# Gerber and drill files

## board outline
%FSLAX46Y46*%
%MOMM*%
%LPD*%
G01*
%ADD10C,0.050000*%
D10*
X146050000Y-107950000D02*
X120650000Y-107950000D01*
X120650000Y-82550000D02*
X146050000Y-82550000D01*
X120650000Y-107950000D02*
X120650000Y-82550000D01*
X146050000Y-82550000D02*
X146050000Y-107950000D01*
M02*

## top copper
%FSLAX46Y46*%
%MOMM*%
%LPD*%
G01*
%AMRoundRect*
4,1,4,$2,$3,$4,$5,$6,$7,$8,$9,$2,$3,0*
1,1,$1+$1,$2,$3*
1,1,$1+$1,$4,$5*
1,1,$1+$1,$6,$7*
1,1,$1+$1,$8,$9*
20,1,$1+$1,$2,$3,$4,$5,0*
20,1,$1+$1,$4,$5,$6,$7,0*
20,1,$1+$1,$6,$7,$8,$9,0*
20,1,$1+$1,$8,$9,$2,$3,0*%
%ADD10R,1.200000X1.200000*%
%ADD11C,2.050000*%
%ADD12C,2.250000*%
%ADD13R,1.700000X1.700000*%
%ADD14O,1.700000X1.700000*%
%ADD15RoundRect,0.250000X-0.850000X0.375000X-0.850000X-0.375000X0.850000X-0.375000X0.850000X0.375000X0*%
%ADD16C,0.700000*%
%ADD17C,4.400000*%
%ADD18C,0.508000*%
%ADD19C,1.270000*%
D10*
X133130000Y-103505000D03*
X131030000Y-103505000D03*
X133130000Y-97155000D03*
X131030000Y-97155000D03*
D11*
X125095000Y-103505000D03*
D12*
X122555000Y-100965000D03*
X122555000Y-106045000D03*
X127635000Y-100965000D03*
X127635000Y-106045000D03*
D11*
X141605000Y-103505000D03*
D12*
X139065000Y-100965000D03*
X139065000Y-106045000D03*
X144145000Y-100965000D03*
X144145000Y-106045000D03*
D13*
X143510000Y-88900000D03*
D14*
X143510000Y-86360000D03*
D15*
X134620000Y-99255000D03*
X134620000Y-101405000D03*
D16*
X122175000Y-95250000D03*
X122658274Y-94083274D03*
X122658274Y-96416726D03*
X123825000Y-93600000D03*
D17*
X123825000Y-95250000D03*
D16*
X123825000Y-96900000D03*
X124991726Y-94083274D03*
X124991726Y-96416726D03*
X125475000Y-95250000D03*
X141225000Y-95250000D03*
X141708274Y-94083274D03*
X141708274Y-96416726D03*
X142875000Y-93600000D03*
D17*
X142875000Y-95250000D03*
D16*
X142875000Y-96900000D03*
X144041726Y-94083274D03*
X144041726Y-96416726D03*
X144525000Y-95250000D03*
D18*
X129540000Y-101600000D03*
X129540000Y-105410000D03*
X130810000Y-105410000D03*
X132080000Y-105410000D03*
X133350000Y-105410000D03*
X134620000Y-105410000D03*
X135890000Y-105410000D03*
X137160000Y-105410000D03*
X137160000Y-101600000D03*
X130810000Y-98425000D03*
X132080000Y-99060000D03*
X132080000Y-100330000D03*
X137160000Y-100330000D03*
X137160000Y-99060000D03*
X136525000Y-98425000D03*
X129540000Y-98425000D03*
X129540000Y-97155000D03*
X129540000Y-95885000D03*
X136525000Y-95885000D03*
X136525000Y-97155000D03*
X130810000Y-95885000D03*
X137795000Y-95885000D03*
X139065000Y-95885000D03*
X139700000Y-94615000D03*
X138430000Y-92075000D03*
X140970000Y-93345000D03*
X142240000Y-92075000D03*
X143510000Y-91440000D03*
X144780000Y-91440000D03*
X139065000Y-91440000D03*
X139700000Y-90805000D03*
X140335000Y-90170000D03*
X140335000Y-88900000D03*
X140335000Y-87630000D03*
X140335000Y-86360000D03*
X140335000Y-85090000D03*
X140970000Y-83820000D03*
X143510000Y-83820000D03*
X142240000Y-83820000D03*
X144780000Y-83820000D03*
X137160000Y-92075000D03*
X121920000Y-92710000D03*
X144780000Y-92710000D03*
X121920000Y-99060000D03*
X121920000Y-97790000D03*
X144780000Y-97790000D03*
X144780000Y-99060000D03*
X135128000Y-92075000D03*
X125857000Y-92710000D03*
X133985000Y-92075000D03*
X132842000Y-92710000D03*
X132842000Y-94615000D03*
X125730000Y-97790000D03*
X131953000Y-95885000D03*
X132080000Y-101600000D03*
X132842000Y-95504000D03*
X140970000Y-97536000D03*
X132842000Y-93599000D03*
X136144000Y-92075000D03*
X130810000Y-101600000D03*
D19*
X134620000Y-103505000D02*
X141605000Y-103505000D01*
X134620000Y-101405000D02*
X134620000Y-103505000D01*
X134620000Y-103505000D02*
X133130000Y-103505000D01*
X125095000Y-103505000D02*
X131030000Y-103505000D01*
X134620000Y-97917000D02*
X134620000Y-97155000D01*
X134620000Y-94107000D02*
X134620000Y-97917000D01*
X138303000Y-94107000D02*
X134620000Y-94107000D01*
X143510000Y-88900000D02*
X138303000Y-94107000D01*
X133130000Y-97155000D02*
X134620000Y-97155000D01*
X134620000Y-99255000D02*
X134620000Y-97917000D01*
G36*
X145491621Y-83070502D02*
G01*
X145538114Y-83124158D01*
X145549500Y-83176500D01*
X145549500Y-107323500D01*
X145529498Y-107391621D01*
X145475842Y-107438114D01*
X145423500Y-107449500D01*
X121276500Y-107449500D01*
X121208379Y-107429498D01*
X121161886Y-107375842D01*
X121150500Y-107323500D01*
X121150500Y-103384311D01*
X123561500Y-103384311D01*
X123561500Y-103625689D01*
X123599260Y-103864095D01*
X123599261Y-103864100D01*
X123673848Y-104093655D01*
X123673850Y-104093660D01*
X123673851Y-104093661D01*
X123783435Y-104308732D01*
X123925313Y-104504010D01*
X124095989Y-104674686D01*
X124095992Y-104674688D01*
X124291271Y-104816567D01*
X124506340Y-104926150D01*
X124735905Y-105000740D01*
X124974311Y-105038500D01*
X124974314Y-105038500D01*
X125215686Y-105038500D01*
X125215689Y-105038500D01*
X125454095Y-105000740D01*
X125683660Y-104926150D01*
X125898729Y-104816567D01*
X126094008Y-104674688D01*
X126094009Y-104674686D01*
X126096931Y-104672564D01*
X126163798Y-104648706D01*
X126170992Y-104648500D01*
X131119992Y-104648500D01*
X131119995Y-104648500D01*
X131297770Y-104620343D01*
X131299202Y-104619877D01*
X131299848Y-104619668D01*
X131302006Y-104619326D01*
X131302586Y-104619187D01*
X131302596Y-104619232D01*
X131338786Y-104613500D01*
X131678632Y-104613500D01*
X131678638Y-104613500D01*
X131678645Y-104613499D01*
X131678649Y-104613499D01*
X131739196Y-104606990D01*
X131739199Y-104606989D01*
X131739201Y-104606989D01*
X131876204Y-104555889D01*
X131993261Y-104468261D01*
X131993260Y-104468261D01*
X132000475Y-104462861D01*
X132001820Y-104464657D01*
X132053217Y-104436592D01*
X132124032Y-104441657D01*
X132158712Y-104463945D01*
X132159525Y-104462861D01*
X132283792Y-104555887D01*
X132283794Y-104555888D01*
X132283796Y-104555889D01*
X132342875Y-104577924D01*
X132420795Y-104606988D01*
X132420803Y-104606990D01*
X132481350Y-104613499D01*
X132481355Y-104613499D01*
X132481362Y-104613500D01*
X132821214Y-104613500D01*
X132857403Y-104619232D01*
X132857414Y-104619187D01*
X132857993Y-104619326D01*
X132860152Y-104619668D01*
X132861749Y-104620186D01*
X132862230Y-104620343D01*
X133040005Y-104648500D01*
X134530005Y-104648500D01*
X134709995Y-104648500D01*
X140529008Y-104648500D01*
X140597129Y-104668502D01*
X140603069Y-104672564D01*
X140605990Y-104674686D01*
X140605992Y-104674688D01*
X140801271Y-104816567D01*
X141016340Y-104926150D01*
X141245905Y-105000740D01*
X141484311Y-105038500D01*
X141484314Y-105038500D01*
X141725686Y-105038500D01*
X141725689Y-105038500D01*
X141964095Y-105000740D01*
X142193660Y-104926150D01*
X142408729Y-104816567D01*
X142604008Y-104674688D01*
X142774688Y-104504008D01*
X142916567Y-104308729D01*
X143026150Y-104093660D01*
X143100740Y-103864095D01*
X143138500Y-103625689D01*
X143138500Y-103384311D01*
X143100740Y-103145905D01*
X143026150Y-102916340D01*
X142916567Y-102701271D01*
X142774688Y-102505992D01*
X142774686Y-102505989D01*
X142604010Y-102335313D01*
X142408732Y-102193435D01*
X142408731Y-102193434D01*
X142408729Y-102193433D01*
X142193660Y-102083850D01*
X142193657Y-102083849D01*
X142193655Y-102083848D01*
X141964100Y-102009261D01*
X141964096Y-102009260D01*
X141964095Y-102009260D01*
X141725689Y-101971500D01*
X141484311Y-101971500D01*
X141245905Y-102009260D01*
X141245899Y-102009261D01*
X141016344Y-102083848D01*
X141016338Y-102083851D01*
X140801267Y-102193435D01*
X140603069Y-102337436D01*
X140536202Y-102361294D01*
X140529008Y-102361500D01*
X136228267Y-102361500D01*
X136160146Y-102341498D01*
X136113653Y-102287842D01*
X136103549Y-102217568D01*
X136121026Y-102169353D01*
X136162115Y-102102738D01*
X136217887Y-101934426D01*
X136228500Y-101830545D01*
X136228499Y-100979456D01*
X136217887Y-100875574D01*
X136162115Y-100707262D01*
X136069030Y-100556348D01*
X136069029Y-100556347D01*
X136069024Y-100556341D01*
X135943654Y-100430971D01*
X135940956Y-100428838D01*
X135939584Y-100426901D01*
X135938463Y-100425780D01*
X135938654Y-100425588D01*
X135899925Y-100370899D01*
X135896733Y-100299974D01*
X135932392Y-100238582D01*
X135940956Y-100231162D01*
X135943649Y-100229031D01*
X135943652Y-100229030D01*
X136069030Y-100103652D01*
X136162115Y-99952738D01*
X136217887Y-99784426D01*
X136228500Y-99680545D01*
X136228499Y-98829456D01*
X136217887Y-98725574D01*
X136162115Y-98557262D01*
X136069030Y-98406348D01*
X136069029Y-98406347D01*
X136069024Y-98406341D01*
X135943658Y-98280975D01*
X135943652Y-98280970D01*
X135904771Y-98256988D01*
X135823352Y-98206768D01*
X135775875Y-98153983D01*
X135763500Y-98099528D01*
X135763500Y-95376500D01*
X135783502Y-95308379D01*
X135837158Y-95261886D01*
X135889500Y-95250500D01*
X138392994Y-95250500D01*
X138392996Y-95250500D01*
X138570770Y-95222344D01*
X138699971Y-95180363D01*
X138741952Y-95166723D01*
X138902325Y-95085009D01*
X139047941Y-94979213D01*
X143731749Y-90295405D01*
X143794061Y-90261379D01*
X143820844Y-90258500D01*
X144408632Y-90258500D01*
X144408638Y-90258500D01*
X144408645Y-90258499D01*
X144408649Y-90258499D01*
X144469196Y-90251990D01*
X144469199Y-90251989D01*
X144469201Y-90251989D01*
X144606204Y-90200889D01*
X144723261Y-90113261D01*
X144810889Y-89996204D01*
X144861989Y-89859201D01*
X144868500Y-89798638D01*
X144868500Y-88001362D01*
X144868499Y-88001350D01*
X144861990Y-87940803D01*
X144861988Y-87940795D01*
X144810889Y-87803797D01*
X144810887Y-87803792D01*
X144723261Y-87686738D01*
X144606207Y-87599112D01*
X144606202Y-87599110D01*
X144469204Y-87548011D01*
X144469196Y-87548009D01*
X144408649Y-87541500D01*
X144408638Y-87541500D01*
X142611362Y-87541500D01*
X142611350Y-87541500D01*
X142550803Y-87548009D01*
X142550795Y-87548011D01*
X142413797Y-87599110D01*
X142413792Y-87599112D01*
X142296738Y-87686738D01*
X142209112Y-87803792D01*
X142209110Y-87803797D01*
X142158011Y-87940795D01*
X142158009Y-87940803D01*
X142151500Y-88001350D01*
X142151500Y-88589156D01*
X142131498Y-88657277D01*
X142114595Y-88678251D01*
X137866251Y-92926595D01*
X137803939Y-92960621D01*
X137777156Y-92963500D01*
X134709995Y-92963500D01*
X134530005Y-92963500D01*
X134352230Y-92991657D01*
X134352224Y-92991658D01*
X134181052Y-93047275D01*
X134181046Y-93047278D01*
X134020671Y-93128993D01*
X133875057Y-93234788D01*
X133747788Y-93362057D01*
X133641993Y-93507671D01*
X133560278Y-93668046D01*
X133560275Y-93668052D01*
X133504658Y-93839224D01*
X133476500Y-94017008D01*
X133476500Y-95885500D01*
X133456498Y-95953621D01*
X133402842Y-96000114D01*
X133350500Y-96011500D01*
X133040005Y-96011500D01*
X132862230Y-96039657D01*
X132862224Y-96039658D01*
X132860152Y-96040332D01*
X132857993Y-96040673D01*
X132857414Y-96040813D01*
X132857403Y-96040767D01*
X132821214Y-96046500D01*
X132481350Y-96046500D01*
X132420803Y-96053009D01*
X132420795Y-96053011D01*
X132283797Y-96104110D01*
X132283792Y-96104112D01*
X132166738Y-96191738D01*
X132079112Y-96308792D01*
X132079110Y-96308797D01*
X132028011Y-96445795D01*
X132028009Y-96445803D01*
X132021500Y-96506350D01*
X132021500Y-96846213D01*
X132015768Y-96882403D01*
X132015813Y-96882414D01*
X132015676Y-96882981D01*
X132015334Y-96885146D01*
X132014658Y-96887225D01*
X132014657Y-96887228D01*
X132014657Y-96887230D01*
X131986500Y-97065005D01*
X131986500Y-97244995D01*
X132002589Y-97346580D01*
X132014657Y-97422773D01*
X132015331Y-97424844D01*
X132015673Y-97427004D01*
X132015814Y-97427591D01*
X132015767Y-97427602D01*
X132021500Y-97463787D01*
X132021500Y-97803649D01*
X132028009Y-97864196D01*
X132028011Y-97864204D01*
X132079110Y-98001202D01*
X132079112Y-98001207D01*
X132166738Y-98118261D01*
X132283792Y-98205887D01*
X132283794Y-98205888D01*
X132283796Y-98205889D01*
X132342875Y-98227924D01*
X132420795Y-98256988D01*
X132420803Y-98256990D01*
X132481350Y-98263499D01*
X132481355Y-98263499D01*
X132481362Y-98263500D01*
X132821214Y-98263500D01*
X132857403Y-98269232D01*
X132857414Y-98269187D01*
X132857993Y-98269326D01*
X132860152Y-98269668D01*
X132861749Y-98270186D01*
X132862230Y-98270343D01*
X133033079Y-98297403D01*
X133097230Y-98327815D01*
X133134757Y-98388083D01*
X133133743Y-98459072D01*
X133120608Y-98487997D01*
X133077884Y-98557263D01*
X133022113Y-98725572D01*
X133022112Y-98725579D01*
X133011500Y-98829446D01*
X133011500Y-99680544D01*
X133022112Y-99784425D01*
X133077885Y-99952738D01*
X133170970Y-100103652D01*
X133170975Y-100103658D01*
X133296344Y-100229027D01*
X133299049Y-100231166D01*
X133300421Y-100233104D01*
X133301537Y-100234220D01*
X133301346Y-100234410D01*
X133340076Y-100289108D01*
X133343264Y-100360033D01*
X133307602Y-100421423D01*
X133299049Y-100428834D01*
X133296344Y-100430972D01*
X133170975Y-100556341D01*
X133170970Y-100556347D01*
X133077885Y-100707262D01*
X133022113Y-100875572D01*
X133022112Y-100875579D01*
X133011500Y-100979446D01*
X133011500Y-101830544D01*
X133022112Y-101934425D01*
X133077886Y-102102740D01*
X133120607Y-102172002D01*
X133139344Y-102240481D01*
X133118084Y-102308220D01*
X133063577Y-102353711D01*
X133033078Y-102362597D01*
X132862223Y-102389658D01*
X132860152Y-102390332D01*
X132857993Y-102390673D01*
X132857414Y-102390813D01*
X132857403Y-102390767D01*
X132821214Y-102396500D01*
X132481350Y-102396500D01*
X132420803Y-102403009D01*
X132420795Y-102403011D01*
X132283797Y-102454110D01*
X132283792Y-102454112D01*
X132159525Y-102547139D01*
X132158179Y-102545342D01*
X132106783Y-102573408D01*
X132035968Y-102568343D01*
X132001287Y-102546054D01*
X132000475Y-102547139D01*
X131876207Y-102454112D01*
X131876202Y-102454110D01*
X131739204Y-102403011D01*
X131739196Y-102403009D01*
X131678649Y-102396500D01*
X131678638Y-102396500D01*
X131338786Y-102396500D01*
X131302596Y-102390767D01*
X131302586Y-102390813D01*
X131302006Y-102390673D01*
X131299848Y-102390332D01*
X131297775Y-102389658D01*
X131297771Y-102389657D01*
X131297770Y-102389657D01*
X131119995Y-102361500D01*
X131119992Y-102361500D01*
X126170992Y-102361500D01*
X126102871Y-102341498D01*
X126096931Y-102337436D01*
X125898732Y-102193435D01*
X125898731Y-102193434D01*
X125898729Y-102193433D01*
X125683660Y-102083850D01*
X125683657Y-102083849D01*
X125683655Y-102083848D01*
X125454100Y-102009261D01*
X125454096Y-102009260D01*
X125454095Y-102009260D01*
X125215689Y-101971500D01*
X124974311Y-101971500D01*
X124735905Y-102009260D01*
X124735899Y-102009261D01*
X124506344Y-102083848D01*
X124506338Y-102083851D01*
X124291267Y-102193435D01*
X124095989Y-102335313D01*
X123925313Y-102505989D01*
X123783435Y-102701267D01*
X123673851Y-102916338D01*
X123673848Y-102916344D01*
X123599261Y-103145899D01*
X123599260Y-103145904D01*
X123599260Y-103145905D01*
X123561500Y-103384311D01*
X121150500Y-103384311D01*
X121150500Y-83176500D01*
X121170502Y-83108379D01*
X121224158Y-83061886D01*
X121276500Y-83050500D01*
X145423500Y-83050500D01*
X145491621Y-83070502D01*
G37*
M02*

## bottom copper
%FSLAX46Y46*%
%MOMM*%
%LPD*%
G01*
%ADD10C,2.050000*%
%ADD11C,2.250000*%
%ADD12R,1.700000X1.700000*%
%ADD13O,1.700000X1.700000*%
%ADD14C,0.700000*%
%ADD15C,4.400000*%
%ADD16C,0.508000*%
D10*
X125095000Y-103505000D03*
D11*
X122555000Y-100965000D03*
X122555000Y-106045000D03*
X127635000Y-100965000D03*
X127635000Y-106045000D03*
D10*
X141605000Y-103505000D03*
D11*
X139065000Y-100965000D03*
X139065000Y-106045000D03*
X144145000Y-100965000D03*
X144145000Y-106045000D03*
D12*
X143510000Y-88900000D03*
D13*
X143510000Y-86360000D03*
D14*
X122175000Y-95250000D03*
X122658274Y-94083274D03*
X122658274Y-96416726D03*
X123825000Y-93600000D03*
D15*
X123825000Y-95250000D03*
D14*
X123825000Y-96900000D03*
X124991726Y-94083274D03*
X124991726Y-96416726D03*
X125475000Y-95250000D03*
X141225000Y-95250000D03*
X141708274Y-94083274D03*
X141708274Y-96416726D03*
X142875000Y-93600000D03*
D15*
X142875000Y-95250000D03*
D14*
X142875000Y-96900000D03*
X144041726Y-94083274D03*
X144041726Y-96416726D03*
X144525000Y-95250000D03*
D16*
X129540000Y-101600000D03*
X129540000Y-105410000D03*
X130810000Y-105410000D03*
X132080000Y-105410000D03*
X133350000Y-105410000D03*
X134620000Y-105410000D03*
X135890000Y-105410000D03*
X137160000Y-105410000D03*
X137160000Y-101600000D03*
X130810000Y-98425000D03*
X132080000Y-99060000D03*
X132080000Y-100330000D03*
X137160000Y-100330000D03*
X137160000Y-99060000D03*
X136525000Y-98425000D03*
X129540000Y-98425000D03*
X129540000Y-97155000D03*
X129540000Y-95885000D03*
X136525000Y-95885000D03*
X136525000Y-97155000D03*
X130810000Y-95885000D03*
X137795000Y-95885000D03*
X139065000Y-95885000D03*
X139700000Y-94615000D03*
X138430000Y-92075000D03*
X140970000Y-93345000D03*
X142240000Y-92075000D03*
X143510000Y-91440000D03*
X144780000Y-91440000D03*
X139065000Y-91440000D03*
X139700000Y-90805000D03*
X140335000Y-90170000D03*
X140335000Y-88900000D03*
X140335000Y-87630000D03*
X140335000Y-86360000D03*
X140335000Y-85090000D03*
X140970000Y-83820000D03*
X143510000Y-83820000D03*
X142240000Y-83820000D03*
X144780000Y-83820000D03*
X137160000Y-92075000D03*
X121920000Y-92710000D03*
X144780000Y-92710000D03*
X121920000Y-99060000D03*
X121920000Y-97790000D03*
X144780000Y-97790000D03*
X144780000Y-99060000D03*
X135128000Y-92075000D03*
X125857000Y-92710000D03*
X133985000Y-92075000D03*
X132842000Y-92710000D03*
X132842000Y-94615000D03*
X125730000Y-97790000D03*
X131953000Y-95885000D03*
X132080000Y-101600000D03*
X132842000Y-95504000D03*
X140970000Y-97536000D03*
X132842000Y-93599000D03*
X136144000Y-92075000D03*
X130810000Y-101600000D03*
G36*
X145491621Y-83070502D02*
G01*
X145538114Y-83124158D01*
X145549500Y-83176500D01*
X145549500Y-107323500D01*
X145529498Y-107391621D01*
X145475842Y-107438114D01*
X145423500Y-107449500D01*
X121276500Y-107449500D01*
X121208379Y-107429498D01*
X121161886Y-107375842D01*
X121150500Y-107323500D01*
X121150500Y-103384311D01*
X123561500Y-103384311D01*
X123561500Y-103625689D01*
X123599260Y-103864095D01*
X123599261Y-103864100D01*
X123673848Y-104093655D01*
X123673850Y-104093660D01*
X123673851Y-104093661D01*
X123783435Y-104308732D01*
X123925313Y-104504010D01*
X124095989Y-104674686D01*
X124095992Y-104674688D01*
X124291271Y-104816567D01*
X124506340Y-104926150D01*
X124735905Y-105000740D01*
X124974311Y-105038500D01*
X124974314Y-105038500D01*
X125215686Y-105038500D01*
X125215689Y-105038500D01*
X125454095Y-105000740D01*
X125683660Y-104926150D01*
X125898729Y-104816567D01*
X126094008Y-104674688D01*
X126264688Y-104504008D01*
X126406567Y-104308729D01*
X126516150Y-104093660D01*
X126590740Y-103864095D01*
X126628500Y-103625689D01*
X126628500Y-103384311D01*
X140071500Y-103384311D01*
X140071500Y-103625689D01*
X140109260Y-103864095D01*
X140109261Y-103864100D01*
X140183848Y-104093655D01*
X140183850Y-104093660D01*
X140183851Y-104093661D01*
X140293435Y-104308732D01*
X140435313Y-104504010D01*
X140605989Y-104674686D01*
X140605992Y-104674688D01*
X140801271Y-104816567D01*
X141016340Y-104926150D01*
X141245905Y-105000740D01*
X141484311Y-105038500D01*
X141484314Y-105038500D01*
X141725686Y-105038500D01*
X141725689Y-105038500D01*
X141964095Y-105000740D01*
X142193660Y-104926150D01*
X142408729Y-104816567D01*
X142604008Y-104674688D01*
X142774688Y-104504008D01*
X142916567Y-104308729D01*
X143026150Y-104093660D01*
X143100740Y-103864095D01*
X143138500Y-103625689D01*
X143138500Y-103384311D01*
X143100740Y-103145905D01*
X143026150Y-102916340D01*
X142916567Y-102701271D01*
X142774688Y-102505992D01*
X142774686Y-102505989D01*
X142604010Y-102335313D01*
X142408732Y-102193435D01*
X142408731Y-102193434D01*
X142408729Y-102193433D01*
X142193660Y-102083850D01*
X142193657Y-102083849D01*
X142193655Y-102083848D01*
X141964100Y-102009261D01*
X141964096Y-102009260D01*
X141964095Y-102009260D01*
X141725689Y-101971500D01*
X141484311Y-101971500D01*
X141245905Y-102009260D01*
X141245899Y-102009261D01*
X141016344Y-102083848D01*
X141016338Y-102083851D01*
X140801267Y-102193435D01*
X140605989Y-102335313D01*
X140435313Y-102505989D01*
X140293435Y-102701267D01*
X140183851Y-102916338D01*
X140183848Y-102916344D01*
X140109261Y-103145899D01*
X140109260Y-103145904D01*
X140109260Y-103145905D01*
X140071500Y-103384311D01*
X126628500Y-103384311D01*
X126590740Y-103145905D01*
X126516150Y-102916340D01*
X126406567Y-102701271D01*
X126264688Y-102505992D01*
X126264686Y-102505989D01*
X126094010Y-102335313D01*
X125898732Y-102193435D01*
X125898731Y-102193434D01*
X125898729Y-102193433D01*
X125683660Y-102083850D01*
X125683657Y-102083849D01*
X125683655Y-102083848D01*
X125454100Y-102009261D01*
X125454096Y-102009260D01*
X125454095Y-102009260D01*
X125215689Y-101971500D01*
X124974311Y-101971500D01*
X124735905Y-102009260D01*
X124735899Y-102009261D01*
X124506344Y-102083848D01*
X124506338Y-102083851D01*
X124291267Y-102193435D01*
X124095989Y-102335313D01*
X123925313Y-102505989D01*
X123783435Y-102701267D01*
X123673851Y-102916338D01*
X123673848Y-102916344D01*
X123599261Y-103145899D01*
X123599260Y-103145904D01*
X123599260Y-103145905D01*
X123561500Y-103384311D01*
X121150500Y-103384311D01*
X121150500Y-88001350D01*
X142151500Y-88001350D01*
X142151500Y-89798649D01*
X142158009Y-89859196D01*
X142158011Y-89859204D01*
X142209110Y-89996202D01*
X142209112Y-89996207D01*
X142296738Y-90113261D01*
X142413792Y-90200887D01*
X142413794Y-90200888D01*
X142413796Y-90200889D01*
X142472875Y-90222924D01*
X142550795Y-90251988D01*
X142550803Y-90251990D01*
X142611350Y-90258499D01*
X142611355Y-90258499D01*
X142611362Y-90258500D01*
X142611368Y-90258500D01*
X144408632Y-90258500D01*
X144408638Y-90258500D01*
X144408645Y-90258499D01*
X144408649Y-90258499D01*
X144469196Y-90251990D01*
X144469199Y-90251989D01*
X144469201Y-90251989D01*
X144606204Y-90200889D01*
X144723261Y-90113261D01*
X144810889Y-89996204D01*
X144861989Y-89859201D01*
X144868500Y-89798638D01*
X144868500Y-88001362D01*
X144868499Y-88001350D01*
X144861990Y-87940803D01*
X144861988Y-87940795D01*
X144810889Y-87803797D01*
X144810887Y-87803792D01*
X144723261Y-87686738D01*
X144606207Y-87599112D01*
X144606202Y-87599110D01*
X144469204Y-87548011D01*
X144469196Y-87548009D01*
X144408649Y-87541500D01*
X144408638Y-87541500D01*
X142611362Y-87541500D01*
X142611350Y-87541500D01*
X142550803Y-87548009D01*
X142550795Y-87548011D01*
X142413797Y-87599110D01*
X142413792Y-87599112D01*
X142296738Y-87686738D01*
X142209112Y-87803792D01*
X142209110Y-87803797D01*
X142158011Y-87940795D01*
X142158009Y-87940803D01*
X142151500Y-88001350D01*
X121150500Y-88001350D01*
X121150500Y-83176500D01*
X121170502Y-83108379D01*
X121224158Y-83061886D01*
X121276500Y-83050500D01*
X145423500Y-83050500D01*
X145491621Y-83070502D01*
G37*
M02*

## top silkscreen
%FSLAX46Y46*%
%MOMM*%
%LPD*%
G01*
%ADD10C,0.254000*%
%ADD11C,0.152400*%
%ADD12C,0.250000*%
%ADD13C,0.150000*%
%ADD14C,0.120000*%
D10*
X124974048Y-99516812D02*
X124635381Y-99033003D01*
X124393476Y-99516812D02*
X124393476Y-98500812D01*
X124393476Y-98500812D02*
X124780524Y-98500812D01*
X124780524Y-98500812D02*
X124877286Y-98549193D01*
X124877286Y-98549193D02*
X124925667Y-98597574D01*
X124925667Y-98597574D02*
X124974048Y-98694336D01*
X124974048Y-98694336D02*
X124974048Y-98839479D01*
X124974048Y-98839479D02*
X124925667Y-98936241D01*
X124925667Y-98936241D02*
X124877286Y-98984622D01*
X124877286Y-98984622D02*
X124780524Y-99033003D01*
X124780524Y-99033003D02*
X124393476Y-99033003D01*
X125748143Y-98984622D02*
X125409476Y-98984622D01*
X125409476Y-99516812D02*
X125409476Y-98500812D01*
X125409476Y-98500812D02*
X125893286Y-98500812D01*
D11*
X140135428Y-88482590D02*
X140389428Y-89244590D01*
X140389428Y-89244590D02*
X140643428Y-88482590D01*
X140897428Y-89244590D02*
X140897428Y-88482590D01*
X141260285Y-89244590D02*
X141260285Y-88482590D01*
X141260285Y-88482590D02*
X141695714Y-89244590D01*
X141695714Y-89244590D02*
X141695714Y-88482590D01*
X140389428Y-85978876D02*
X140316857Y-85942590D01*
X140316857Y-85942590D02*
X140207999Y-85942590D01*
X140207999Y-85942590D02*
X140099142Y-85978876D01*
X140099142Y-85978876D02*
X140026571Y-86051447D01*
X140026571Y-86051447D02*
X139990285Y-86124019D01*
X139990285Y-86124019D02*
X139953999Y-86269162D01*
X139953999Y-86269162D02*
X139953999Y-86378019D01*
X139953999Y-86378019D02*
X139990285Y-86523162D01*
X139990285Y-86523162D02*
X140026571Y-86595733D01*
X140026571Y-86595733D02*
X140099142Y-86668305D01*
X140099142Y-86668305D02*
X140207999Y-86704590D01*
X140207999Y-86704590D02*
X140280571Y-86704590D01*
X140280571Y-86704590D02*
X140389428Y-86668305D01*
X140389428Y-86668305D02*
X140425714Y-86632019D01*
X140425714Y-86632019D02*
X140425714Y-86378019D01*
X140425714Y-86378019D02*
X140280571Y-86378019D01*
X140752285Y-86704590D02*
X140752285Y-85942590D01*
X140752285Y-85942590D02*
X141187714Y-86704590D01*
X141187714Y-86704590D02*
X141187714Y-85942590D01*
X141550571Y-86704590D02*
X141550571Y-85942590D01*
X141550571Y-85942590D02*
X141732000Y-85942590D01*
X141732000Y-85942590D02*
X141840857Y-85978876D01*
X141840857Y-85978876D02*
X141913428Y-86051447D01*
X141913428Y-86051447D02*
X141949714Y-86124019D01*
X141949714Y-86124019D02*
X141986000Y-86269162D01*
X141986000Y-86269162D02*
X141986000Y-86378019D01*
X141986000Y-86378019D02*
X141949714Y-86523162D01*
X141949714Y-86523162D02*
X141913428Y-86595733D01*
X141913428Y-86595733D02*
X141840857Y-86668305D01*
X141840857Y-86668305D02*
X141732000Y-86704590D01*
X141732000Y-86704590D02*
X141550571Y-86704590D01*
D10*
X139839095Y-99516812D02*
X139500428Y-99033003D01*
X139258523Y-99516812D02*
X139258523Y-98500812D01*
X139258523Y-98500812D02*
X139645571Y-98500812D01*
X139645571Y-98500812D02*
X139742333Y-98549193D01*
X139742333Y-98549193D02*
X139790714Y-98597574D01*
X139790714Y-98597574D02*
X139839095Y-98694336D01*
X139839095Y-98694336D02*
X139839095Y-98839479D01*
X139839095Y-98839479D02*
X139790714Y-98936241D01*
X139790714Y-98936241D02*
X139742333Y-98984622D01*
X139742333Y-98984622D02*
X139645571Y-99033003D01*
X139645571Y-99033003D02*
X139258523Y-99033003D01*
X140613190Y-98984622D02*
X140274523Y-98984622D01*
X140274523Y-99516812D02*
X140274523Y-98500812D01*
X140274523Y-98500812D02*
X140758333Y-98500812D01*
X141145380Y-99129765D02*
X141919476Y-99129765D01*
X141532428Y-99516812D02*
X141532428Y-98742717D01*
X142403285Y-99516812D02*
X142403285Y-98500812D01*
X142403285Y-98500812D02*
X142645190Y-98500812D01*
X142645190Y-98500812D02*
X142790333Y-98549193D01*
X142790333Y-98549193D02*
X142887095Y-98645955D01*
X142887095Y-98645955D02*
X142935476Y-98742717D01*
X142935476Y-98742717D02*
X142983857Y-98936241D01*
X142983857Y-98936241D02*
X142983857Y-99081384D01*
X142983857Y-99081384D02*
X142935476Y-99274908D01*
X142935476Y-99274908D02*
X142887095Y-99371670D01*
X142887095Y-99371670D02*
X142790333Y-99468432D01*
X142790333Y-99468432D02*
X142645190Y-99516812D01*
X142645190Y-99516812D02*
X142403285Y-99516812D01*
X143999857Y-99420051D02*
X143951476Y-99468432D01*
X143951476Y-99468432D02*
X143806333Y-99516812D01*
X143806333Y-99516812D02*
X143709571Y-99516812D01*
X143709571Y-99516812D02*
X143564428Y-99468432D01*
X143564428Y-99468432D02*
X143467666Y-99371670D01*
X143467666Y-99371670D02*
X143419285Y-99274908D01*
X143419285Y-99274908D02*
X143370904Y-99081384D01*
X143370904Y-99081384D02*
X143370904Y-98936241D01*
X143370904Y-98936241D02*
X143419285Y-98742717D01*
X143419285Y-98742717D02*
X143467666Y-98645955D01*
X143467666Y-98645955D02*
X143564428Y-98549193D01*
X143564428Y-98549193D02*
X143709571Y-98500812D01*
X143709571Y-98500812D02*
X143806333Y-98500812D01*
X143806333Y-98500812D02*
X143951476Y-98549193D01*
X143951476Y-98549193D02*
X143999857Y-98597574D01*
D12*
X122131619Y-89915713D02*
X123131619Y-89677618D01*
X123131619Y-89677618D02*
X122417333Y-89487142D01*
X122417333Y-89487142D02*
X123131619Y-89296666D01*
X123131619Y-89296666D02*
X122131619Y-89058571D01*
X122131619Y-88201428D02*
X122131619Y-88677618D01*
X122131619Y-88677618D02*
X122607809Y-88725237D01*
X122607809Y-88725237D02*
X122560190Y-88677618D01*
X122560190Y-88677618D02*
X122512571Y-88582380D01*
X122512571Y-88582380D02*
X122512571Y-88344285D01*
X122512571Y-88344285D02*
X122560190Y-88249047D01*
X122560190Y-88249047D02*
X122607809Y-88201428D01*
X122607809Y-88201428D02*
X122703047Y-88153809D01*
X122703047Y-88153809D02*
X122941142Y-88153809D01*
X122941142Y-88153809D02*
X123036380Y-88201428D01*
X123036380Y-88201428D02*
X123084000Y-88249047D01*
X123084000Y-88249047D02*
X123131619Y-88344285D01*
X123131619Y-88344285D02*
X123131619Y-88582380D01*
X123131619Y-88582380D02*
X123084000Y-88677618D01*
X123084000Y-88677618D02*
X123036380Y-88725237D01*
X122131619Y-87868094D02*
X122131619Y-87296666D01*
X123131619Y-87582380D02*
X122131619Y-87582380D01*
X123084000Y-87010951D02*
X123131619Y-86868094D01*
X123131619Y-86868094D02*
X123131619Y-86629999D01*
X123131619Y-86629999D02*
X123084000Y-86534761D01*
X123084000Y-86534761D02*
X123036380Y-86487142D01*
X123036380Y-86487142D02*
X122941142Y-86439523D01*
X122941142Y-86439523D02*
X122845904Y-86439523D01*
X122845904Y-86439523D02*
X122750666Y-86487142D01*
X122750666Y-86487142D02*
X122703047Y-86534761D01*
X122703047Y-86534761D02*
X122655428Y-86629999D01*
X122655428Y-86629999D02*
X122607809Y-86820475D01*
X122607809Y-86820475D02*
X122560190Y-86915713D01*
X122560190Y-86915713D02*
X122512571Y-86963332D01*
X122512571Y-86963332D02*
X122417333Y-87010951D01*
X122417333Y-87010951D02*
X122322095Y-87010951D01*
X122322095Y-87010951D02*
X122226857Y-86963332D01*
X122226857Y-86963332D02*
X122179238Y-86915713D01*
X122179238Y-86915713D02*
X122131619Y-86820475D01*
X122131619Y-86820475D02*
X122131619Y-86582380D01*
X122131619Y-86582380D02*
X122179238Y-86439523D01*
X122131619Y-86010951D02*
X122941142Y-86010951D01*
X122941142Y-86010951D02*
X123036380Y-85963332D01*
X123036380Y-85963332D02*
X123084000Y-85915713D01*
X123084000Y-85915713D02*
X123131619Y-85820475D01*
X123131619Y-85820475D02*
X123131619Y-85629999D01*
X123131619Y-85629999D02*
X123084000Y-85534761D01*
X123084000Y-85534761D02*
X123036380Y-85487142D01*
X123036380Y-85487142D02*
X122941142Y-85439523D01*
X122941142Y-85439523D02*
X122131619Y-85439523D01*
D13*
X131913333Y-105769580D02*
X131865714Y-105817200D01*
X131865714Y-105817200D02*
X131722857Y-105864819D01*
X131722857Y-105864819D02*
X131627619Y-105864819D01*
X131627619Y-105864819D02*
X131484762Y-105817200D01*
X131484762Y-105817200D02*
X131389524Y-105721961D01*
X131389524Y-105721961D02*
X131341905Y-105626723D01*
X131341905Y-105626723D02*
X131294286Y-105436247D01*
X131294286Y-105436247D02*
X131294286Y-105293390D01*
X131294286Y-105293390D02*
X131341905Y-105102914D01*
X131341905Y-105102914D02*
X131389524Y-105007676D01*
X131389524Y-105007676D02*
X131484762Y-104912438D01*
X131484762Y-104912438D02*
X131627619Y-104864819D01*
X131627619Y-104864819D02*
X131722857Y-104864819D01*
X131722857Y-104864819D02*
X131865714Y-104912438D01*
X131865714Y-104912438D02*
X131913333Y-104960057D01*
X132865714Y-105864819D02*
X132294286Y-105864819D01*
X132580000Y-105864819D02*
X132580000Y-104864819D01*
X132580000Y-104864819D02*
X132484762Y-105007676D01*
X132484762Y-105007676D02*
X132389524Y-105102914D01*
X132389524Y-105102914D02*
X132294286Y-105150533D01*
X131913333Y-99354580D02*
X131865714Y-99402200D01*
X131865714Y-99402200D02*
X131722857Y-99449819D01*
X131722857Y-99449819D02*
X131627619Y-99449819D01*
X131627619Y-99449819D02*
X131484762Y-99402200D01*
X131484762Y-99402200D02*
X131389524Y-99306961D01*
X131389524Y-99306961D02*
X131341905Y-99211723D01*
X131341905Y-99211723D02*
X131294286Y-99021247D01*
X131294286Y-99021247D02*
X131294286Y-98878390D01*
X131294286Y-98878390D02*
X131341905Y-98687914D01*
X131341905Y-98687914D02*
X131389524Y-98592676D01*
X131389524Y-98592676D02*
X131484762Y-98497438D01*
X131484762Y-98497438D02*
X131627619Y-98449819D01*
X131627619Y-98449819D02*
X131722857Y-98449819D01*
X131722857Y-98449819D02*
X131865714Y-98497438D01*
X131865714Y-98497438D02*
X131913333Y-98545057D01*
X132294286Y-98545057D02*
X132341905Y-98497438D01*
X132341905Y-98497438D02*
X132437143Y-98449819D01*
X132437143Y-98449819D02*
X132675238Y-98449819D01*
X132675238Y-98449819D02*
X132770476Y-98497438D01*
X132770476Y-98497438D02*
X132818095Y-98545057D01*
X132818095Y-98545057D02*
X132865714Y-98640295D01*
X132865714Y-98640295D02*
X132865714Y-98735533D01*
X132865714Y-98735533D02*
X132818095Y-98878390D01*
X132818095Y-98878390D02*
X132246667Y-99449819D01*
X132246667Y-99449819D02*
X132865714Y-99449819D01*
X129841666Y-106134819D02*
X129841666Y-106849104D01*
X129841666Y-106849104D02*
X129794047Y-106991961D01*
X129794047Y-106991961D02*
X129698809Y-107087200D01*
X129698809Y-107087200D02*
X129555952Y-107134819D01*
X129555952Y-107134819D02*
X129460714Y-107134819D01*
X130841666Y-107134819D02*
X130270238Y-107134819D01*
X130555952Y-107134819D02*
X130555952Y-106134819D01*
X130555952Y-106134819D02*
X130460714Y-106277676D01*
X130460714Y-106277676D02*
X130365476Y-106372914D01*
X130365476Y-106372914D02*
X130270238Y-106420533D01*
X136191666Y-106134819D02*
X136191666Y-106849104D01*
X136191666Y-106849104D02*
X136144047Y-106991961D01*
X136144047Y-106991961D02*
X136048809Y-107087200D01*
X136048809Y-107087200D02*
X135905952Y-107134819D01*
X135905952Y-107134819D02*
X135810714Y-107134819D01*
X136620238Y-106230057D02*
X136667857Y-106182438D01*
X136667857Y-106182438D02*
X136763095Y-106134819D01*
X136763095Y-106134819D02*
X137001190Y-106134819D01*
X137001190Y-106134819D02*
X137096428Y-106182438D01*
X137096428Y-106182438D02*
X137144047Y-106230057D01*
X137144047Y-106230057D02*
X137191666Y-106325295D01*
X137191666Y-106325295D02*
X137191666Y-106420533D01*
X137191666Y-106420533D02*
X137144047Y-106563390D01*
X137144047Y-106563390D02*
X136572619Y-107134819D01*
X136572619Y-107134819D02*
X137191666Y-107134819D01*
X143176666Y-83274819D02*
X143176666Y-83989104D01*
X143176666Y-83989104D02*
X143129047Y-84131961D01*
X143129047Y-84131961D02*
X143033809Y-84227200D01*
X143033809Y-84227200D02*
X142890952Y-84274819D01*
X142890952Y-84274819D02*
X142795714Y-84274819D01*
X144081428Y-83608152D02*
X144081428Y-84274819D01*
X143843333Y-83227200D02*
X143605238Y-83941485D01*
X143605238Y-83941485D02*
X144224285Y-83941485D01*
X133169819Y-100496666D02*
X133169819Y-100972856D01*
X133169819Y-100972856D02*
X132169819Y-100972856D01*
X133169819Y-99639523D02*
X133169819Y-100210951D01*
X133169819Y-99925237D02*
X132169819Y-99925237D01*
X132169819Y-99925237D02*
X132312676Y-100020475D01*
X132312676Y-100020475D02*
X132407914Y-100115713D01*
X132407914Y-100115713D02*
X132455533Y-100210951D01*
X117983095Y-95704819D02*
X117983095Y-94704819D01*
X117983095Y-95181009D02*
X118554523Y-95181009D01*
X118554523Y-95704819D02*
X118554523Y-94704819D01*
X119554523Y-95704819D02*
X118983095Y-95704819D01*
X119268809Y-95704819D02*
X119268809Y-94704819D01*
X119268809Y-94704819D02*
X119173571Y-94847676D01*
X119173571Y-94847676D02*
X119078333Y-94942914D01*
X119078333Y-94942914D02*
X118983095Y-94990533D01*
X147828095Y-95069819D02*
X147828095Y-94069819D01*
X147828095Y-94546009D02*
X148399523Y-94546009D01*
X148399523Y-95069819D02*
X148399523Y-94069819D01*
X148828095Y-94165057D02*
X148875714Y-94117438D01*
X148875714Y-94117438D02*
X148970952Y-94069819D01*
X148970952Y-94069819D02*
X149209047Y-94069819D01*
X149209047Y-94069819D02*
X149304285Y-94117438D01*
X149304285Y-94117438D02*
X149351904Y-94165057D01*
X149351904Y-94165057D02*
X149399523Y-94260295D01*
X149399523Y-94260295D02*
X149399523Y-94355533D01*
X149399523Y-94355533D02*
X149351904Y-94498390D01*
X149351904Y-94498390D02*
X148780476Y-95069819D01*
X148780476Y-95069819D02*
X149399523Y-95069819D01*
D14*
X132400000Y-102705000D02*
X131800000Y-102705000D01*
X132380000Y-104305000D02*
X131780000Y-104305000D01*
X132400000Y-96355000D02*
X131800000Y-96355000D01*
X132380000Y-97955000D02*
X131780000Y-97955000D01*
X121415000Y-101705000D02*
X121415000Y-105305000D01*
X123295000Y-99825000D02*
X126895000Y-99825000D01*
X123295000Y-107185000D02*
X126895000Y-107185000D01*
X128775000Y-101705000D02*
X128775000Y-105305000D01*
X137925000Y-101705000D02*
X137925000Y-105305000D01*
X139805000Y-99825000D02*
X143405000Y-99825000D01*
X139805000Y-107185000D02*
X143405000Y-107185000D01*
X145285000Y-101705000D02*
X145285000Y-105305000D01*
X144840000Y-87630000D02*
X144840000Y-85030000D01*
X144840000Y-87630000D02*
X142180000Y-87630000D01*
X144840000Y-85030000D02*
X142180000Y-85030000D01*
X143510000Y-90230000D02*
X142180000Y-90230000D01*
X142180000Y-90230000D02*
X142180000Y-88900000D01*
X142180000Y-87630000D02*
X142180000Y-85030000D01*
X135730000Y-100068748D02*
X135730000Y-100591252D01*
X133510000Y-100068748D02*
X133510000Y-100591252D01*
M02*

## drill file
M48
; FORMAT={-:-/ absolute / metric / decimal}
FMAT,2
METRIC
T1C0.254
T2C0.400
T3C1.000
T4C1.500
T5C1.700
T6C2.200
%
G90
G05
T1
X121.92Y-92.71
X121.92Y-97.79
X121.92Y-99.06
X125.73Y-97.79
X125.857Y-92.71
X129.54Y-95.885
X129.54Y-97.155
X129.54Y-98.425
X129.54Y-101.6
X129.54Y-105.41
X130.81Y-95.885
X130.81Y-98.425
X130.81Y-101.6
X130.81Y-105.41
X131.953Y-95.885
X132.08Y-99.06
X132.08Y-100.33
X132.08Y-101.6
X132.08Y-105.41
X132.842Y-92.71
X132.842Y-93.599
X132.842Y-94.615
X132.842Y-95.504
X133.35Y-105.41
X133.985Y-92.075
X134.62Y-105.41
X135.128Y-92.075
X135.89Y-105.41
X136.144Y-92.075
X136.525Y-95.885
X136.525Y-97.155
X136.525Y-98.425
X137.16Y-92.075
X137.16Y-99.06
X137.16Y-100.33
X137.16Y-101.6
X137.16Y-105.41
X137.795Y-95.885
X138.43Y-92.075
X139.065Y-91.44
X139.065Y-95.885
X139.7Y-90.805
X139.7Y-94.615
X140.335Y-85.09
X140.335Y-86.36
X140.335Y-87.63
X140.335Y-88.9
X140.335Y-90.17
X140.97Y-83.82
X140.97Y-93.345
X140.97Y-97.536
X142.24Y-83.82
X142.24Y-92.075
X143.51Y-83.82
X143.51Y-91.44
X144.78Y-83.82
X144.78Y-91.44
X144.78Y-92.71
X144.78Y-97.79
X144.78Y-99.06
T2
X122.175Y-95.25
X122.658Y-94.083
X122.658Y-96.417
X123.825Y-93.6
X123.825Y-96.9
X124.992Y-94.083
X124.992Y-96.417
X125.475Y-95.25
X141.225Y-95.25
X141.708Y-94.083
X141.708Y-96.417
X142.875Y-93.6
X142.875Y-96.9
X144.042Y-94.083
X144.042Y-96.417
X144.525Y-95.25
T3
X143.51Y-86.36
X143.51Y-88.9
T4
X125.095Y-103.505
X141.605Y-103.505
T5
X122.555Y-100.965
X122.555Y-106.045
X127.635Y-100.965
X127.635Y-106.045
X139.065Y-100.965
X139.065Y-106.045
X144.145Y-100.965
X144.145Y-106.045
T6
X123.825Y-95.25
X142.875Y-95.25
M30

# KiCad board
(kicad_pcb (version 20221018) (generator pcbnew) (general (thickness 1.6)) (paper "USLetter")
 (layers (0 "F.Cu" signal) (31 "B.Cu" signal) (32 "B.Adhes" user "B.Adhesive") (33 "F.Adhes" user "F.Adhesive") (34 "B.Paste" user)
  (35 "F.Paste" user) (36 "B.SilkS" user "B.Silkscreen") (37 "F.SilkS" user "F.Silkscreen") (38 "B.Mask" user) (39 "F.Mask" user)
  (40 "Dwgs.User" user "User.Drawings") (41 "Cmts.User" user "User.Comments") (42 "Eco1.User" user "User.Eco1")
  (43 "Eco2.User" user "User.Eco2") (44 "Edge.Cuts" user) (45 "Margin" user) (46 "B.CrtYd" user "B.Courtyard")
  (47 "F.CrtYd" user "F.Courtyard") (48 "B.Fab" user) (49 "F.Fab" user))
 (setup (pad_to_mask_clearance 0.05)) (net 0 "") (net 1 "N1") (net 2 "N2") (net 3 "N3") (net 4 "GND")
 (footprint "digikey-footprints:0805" (layer "F.Cu") (at 132.08 103.505 180)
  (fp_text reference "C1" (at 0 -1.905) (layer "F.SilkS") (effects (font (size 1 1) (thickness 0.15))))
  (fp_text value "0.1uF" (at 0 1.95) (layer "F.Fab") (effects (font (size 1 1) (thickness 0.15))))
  (fp_line (start -0.32 0.8) (end 0.28 0.8) (stroke (width 0.12) (type solid)) (layer "F.SilkS"))
  (fp_line (start -0.3 -0.8) (end 0.3 -0.8) (stroke (width 0.12) (type solid)) (layer "F.SilkS"))
  (pad "1" smd rect (at -1.05 0 180) (size 1.2 1.2) (layers "F.Cu" "F.Paste" "F.Mask") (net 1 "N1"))
  (pad "2" smd rect (at 1.05 0 180) (size 1.2 1.2) (layers "F.Cu" "F.Paste" "F.Mask") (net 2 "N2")))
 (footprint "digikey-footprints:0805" (layer "F.Cu") (at 132.08 97.155 180)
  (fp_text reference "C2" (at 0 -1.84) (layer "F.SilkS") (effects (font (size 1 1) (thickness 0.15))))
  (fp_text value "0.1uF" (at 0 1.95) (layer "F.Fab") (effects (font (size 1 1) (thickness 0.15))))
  (fp_line (start -0.32 0.8) (end 0.28 0.8) (stroke (width 0.12) (type solid)) (layer "F.SilkS"))
  (fp_line (start -0.3 -0.8) (end 0.3 -0.8) (stroke (width 0.12) (type solid)) (layer "F.SilkS"))
  (pad "1" smd rect (at -1.05 0 180) (size 1.2 1.2) (layers "F.Cu" "F.Paste" "F.Mask") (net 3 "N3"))
  (pad "2" smd rect (at 1.05 0 180) (size 1.2 1.2) (layers "F.Cu" "F.Paste" "F.Mask") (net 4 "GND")))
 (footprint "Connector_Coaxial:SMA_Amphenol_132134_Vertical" (layer "F.Cu") (at 125.095 103.505)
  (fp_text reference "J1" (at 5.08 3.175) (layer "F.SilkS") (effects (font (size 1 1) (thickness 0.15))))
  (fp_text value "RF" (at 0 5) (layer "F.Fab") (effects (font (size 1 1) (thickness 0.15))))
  (fp_line (start -3.68 -1.8) (end -3.68 1.8) (stroke (width 0.12) (type solid)) (layer "F.SilkS"))
  (fp_line (start -1.8 -3.68) (end 1.8 -3.68) (stroke (width 0.12) (type solid)) (layer "F.SilkS"))
  (fp_line (start -1.8 3.68) (end 1.8 3.68) (stroke (width 0.12) (type solid)) (layer "F.SilkS"))
  (fp_line (start 3.68 -1.8) (end 3.68 1.8) (stroke (width 0.12) (type solid)) (layer "F.SilkS"))
  (pad "1" thru_hole circle (at 0 0) (size 2.05 2.05) (drill 1.5) (layers "*.Cu" "*.Mask") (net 2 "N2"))
  (pad "2" thru_hole circle (at -2.54 -2.54) (size 2.25 2.25) (drill 1.7) (layers "*.Cu" "*.Mask") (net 4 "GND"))
  (pad "2" thru_hole circle (at -2.54 2.54) (size 2.25 2.25) (drill 1.7) (layers "*.Cu" "*.Mask") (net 4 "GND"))
  (pad "2" thru_hole circle (at 2.54 -2.54) (size 2.25 2.25) (drill 1.7) (layers "*.Cu" "*.Mask") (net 4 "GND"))
  (pad "2" thru_hole circle (at 2.54 2.54) (size 2.25 2.25) (drill 1.7) (layers "*.Cu" "*.Mask") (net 4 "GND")))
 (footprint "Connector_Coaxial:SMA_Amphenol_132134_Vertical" (layer "F.Cu") (at 141.605 103.505)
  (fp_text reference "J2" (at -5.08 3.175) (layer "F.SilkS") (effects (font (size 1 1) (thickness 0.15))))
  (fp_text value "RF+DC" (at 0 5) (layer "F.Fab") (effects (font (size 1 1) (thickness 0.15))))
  (fp_line (start -3.68 -1.8) (end -3.68 1.8) (stroke (width 0.12) (type solid)) (layer "F.SilkS"))
  (fp_line (start -1.8 -3.68) (end 1.8 -3.68) (stroke (width 0.12) (type solid)) (layer "F.SilkS"))
  (fp_line (start -1.8 3.68) (end 1.8 3.68) (stroke (width 0.12) (type solid)) (layer "F.SilkS"))
  (fp_line (start 3.68 -1.8) (end 3.68 1.8) (stroke (width 0.12) (type solid)) (layer "F.SilkS"))
  (pad "1" thru_hole circle (at 0 0) (size 2.05 2.05) (drill 1.5) (layers "*.Cu" "*.Mask") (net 1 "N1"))
  (pad "2" thru_hole circle (at -2.54 -2.54) (size 2.25 2.25) (drill 1.7) (layers "*.Cu" "*.Mask") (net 4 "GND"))
  (pad "2" thru_hole circle (at -2.54 2.54) (size 2.25 2.25) (drill 1.7) (layers "*.Cu" "*.Mask") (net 4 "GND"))
  (pad "2" thru_hole circle (at 2.54 -2.54) (size 2.25 2.25) (drill 1.7) (layers "*.Cu" "*.Mask") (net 4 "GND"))
  (pad "2" thru_hole circle (at 2.54 2.54) (size 2.25 2.25) (drill 1.7) (layers "*.Cu" "*.Mask") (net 4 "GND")))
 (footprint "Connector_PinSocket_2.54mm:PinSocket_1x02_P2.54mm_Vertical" (layer "F.Cu") (at 143.51 88.9 180)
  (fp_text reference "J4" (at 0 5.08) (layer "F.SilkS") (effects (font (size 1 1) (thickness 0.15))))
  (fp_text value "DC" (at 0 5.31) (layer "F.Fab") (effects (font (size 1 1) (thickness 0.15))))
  (fp_line (start -1.33 1.27) (end -1.33 3.87) (stroke (width 0.12) (type solid)) (layer "F.SilkS"))
  (fp_line (start -1.33 1.27) (end 1.33 1.27) (stroke (width 0.12) (type solid)) (layer "F.SilkS"))
  (fp_line (start -1.33 3.87) (end 1.33 3.87) (stroke (width 0.12) (type solid)) (layer "F.SilkS"))
  (fp_line (start 0 -1.33) (end 1.33 -1.33) (stroke (width 0.12) (type solid)) (layer "F.SilkS"))
  (fp_line (start 1.33 -1.33) (end 1.33 0) (stroke (width 0.12) (type solid)) (layer "F.SilkS"))
  (fp_line (start 1.33 1.27) (end 1.33 3.87) (stroke (width 0.12) (type solid)) (layer "F.SilkS"))
  (pad "1" thru_hole rect (at 0 0 180) (size 1.7 1.7) (drill 1) (layers "*.Cu" "*.Mask") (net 3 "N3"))
  (pad "2" thru_hole oval (at 0 2.54 180) (size 1.7 1.7) (drill 1) (layers "*.Cu" "*.Mask") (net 4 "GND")))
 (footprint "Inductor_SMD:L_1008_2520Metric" (layer "F.Cu") (at 134.62 100.33 -90)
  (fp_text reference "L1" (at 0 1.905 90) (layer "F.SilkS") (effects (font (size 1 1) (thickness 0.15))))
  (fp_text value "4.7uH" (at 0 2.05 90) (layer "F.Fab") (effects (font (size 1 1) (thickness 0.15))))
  (fp_line (start -0.261252 -1.11) (end 0.261252 -1.11) (stroke (width 0.12) (type solid)) (layer "F.SilkS"))
  (fp_line (start -0.261252 1.11) (end 0.261252 1.11) (stroke (width 0.12) (type solid)) (layer "F.SilkS"))
  (pad "1" smd roundrect (at -1.075 0 270) (size 1.25 2.2) (layers "F.Cu" "F.Paste" "F.Mask") (roundrect_rratio 0.2) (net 3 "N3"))
  (pad "2" smd roundrect (at 1.075 0 270) (size 1.25 2.2) (layers "F.Cu" "F.Paste" "F.Mask") (roundrect_rratio 0.2) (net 1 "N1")))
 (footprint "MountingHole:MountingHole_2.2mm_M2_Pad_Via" (layer "F.Cu") (at 123.825 95.25)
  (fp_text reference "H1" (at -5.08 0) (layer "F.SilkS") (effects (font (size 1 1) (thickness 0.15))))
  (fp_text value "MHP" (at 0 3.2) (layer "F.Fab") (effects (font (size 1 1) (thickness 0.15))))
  (pad "1" thru_hole circle (at -1.65 0) (size 0.7 0.7) (drill 0.4) (layers "*.Cu" "*.Mask") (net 4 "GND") (zone_connect 2))
  (pad "1" thru_hole circle (at -1.166726 -1.166726) (size 0.7 0.7) (drill 0.4) (layers "*.Cu" "*.Mask") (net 4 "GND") (zone_connect 2))
  (pad "1" thru_hole circle (at -1.166726 1.166726) (size 0.7 0.7) (drill 0.4) (layers "*.Cu" "*.Mask") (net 4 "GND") (zone_connect 2))
  (pad "1" thru_hole circle (at 0 -1.65) (size 0.7 0.7) (drill 0.4) (layers "*.Cu" "*.Mask") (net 4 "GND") (zone_connect 2))
  (pad "1" thru_hole circle (at 0 0) (size 4.4 4.4) (drill 2.2) (layers "*.Cu" "*.Mask") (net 4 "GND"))
  (pad "1" thru_hole circle (at 0 1.65) (size 0.7 0.7) (drill 0.4) (layers "*.Cu" "*.Mask") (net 4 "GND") (zone_connect 2))
  (pad "1" thru_hole circle (at 1.166726 -1.166726) (size 0.7 0.7) (drill 0.4) (layers "*.Cu" "*.Mask") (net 4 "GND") (zone_connect 2))
  (pad "1" thru_hole circle (at 1.166726 1.166726) (size 0.7 0.7) (drill 0.4) (layers "*.Cu" "*.Mask") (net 4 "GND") (zone_connect 2))
  (pad "1" thru_hole circle (at 1.65 0) (size 0.7 0.7) (drill 0.4) (layers "*.Cu" "*.Mask") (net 4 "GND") (zone_connect 2)))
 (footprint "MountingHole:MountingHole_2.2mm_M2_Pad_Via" (layer "F.Cu") (at 142.875 95.25)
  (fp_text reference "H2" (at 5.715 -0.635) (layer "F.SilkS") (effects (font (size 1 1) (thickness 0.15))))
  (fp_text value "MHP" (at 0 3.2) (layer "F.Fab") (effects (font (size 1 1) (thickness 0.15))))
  (pad "1" thru_hole circle (at -1.65 0) (size 0.7 0.7) (drill 0.4) (layers "*.Cu" "*.Mask") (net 4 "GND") (zone_connect 2))
  (pad "1" thru_hole circle (at -1.166726 -1.166726) (size 0.7 0.7) (drill 0.4) (layers "*.Cu" "*.Mask") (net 4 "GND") (zone_connect 2))
  (pad "1" thru_hole circle (at -1.166726 1.166726) (size 0.7 0.7) (drill 0.4) (layers "*.Cu" "*.Mask") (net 4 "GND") (zone_connect 2))
  (pad "1" thru_hole circle (at 0 -1.65) (size 0.7 0.7) (drill 0.4) (layers "*.Cu" "*.Mask") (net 4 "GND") (zone_connect 2))
  (pad "1" thru_hole circle (at 0 0) (size 4.4 4.4) (drill 2.2) (layers "*.Cu" "*.Mask") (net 4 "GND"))
  (pad "1" thru_hole circle (at 0 1.65) (size 0.7 0.7) (drill 0.4) (layers "*.Cu" "*.Mask") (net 4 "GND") (zone_connect 2))
  (pad "1" thru_hole circle (at 1.166726 -1.166726) (size 0.7 0.7) (drill 0.4) (layers "*.Cu" "*.Mask") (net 4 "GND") (zone_connect 2))
  (pad "1" thru_hole circle (at 1.166726 1.166726) (size 0.7 0.7) (drill 0.4) (layers "*.Cu" "*.Mask") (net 4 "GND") (zone_connect 2))
  (pad "1" thru_hole circle (at 1.65 0) (size 0.7 0.7) (drill 0.4) (layers "*.Cu" "*.Mask") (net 4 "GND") (zone_connect 2)))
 (gr_line (start 146.05 107.95) (end 120.65 107.95) (stroke (width 0.05) (type solid)) (layer "Edge.Cuts"))
 (gr_line (start 120.65 82.55) (end 146.05 82.55) (stroke (width 0.05) (type solid)) (layer "Edge.Cuts"))
 (gr_line (start 120.65 107.95) (end 120.65 82.55) (stroke (width 0.05) (type solid)) (layer "Edge.Cuts"))
 (gr_line (start 146.05 82.55) (end 146.05 107.95) (stroke (width 0.05) (type solid)) (layer "Edge.Cuts"))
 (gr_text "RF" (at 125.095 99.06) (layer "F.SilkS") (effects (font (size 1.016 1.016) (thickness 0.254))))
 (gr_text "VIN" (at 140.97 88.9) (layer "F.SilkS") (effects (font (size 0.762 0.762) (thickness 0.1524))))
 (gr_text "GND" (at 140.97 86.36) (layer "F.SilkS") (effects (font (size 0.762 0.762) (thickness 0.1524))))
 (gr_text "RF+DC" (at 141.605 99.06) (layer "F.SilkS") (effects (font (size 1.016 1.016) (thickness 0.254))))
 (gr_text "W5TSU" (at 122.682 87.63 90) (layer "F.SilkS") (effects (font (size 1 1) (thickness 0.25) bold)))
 (segment (start 134.62 103.505) (end 141.605 103.505) (width 1.27) (layer "F.Cu") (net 1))
 (segment (start 134.62 101.405) (end 134.62 103.505) (width 1.27) (layer "F.Cu") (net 1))
 (segment (start 134.62 103.505) (end 133.13 103.505) (width 1.27) (layer "F.Cu") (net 1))
 (segment (start 125.095 103.505) (end 131.03 103.505) (width 1.27) (layer "F.Cu") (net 2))
 (via (at 129.54 101.6) (size 0.508) (drill 0.254) (layers "F.Cu" "B.Cu") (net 4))
 (via (at 129.54 105.41) (size 0.508) (drill 0.254) (layers "F.Cu" "B.Cu") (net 4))
 (via (at 130.81 105.41) (size 0.508) (drill 0.254) (layers "F.Cu" "B.Cu") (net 4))
 (via (at 132.08 105.41) (size 0.508) (drill 0.254) (layers "F.Cu" "B.Cu") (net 4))
 (via (at 133.35 105.41) (size 0.508) (drill 0.254) (layers "F.Cu" "B.Cu") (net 4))
 (via (at 134.62 105.41) (size 0.508) (drill 0.254) (layers "F.Cu" "B.Cu") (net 4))
 (via (at 135.89 105.41) (size 0.508) (drill 0.254) (layers "F.Cu" "B.Cu") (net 4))
 (via (at 137.16 105.41) (size 0.508) (drill 0.254) (layers "F.Cu" "B.Cu") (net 4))
 (via (at 137.16 101.6) (size 0.508) (drill 0.254) (layers "F.Cu" "B.Cu") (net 4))
 (via (at 130.81 98.425) (size 0.508) (drill 0.254) (layers "F.Cu" "B.Cu") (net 4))
 (via (at 132.08 99.06) (size 0.508) (drill 0.254) (layers "F.Cu" "B.Cu") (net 4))
 (via (at 132.08 100.33) (size 0.508) (drill 0.254) (layers "F.Cu" "B.Cu") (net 4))
 (via (at 137.16 100.33) (size 0.508) (drill 0.254) (layers "F.Cu" "B.Cu") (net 4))
 (via (at 137.16 99.06) (size 0.508) (drill 0.254) (layers "F.Cu" "B.Cu") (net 4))
 (via (at 136.525 98.425) (size 0.508) (drill 0.254) (layers "F.Cu" "B.Cu") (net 4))
 (via (at 129.54 98.425) (size 0.508) (drill 0.254) (layers "F.Cu" "B.Cu") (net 4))
 (via (at 129.54 97.155) (size 0.508) (drill 0.254) (layers "F.Cu" "B.Cu") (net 4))
 (via (at 129.54 95.885) (size 0.508) (drill 0.254) (layers "F.Cu" "B.Cu") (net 4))
 (via (at 136.525 95.885) (size 0.508) (drill 0.254) (layers "F.Cu" "B.Cu") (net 4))
 (via (at 136.525 97.155) (size 0.508) (drill 0.254) (layers "F.Cu" "B.Cu") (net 4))
 (via (at 130.81 95.885) (size 0.508) (drill 0.254) (layers "F.Cu" "B.Cu") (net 4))
 (via (at 137.795 95.885) (size 0.508) (drill 0.254) (layers "F.Cu" "B.Cu") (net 4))
 (via (at 139.065 95.885) (size 0.508) (drill 0.254) (layers "F.Cu" "B.Cu") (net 4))
 (via (at 139.7 94.615) (size 0.508) (drill 0.254) (layers "F.Cu" "B.Cu") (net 4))
 (via (at 138.43 92.075) (size 0.508) (drill 0.254) (layers "F.Cu" "B.Cu") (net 4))
 (via (at 140.97 93.345) (size 0.508) (drill 0.254) (layers "F.Cu" "B.Cu") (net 4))
 (via (at 142.24 92.075) (size 0.508) (drill 0.254) (layers "F.Cu" "B.Cu") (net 4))
 (via (at 143.51 91.44) (size 0.508) (drill 0.254) (layers "F.Cu" "B.Cu") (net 4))
 (via (at 144.78 91.44) (size 0.508) (drill 0.254) (layers "F.Cu" "B.Cu") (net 4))
 (via (at 139.065 91.44) (size 0.508) (drill 0.254) (layers "F.Cu" "B.Cu") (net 4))
 (via (at 139.7 90.805) (size 0.508) (drill 0.254) (layers "F.Cu" "B.Cu") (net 4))
 (via (at 140.335 90.17) (size 0.508) (drill 0.254) (layers "F.Cu" "B.Cu") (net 4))
 (via (at 140.335 88.9) (size 0.508) (drill 0.254) (layers "F.Cu" "B.Cu") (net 4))
 (via (at 140.335 87.63) (size 0.508) (drill 0.254) (layers "F.Cu" "B.Cu") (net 4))
 (via (at 140.335 86.36) (size 0.508) (drill 0.254) (layers "F.Cu" "B.Cu") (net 4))
 (via (at 140.335 85.09) (size 0.508) (drill 0.254) (layers "F.Cu" "B.Cu") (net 4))
 (via (at 140.97 83.82) (size 0.508) (drill 0.254) (layers "F.Cu" "B.Cu") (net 4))
 (via (at 143.51 83.82) (size 0.508) (drill 0.254) (layers "F.Cu" "B.Cu") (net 4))
 (via (at 142.24 83.82) (size 0.508) (drill 0.254) (layers "F.Cu" "B.Cu") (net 4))
 (via (at 144.78 83.82) (size 0.508) (drill 0.254) (layers "F.Cu" "B.Cu") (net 4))
 (via (at 137.16 92.075) (size 0.508) (drill 0.254) (layers "F.Cu" "B.Cu") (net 4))
 (via (at 121.92 92.71) (size 0.508) (drill 0.254) (layers "F.Cu" "B.Cu") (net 4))
 (via (at 144.78 92.71) (size 0.508) (drill 0.254) (layers "F.Cu" "B.Cu") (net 4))
 (via (at 121.92 99.06) (size 0.508) (drill 0.254) (layers "F.Cu" "B.Cu") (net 4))
 (via (at 121.92 97.79) (size 0.508) (drill 0.254) (layers "F.Cu" "B.Cu") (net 4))
 (via (at 144.78 97.79) (size 0.508) (drill 0.254) (layers "F.Cu" "B.Cu") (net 4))
 (via (at 144.78 99.06) (size 0.508) (drill 0.254) (layers "F.Cu" "B.Cu") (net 4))
 (via (at 135.128 92.075) (size 0.508) (drill 0.254) (layers "F.Cu" "B.Cu") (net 4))
 (via (at 125.857 92.71) (size 0.508) (drill 0.254) (layers "F.Cu" "B.Cu") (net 4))
 (via (at 133.985 92.075) (size 0.508) (drill 0.254) (layers "F.Cu" "B.Cu") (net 4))
 (via (at 132.842 92.71) (size 0.508) (drill 0.254) (layers "F.Cu" "B.Cu") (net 4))
 (via (at 132.842 94.615) (size 0.508) (drill 0.254) (layers "F.Cu" "B.Cu") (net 4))
 (via (at 125.73 97.79) (size 0.508) (drill 0.254) (layers "F.Cu" "B.Cu") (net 4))
 (via (at 131.953 95.885) (size 0.508) (drill 0.254) (layers "F.Cu" "B.Cu") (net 4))
 (via (at 132.08 101.6) (size 0.508) (drill 0.254) (layers "F.Cu" "B.Cu") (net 4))
 (via (at 132.842 95.504) (size 0.508) (drill 0.254) (layers "F.Cu" "B.Cu") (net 4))
 (via (at 140.97 97.536) (size 0.508) (drill 0.254) (layers "F.Cu" "B.Cu") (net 4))
 (via (at 132.842 93.599) (size 0.508) (drill 0.254) (layers "F.Cu" "B.Cu") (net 4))
 (via (at 136.144 92.075) (size 0.508) (drill 0.254) (layers "F.Cu" "B.Cu") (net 4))
 (via (at 130.81 101.6) (size 0.508) (drill 0.254) (layers "F.Cu" "B.Cu") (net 4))
 (segment (start 134.62 97.917) (end 134.62 97.155) (width 1.27) (layer "F.Cu") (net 3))
 (segment (start 134.62 94.107) (end 134.62 97.917) (width 1.27) (layer "F.Cu") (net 3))
 (segment (start 138.303 94.107) (end 134.62 94.107) (width 1.27) (layer "F.Cu") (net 3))
 (segment (start 143.51 88.9) (end 138.303 94.107) (width 1.27) (layer "F.Cu") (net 3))
 (segment (start 133.13 97.155) (end 134.62 97.155) (width 1.27) (layer "F.Cu") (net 3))
 (segment (start 134.62 99.255) (end 134.62 97.917) (width 1.27) (layer "F.Cu") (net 3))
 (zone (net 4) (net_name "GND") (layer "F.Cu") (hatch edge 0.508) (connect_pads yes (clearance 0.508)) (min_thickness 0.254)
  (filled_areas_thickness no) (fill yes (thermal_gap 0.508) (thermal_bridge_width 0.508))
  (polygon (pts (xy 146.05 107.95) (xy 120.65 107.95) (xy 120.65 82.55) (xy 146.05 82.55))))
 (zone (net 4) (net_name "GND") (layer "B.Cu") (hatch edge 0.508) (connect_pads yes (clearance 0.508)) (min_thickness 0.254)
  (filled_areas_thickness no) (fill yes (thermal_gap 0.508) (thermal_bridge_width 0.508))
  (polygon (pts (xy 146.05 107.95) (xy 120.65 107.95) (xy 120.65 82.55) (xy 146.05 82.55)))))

